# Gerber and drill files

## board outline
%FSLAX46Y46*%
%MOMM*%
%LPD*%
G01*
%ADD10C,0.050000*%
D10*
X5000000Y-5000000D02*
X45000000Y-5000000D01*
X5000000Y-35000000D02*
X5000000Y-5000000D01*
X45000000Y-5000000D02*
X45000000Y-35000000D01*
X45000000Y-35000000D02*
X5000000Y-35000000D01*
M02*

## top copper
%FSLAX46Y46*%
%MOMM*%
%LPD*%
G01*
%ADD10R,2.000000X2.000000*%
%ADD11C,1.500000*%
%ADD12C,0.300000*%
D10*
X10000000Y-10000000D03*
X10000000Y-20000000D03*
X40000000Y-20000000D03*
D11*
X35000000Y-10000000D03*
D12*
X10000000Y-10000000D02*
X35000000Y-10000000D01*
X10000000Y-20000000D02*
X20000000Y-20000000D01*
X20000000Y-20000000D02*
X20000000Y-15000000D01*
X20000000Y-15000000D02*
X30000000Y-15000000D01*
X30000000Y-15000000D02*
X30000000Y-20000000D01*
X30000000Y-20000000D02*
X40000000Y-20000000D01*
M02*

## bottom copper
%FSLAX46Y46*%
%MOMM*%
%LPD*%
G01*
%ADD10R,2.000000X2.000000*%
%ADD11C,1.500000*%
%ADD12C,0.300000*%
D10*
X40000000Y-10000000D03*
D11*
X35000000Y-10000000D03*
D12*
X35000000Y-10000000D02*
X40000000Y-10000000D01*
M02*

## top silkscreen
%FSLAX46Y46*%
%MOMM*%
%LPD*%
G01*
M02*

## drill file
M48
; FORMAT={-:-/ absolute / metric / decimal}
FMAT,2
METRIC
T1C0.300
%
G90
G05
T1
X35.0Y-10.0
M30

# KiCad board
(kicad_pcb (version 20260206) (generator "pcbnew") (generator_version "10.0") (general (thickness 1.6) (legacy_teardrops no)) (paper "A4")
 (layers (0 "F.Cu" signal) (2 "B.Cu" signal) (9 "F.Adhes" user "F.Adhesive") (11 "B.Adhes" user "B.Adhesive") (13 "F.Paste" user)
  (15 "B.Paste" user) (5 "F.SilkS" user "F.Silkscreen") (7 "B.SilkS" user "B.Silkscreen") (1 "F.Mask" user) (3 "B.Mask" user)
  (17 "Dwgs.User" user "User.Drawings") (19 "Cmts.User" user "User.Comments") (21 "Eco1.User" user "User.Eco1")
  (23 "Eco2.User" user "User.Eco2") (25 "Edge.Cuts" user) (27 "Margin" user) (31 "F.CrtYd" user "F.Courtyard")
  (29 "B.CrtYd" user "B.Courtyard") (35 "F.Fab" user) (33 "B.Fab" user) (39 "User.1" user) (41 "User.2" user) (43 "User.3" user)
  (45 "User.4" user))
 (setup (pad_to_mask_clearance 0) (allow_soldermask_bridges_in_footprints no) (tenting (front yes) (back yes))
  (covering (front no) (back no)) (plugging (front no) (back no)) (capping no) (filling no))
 (gr_line (start 5 5) (end 45 5) (stroke (width 0.05) (type default)) (layer "Edge.Cuts"))
 (gr_line (start 5 35) (end 5 5) (stroke (width 0.05) (type default)) (layer "Edge.Cuts"))
 (gr_line (start 45 5) (end 45 35) (stroke (width 0.05) (type default)) (layer "Edge.Cuts"))
 (gr_line (start 45 35) (end 5 35) (stroke (width 0.05) (type default)) (layer "Edge.Cuts"))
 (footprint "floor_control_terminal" (layer "F.Cu") (at 10 10)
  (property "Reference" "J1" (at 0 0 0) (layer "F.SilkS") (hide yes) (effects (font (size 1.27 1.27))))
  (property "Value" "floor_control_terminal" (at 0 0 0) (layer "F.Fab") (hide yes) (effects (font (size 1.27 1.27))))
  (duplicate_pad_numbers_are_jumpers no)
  (pad "1" smd rect (at 0 0) (size 2 2) (layers "F.Cu" "F.Paste" "F.Mask") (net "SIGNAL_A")))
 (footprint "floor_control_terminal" (layer "B.Cu") (at 40 10)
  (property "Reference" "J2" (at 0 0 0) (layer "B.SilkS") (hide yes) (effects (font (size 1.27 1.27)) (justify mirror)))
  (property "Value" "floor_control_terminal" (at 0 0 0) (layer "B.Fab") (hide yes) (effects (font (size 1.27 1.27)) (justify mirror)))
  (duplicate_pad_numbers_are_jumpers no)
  (pad "1" smd rect (at 0 0) (size 2 2) (layers "B.Cu" "B.Paste" "B.Mask") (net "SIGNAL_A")))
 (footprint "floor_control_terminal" (layer "F.Cu") (at 10 20)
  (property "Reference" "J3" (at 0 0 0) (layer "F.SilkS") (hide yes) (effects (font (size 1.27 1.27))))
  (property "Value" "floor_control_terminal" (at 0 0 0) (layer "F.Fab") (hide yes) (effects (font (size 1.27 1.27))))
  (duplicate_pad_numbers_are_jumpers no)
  (pad "1" smd rect (at 0 0) (size 2 2) (layers "F.Cu" "F.Paste" "F.Mask") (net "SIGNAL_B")))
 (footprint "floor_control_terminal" (layer "F.Cu") (at 40 20)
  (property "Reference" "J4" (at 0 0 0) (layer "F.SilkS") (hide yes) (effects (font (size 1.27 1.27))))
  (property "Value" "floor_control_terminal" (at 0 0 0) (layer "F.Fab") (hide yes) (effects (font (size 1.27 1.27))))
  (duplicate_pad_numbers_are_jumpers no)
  (pad "1" smd rect (at 0 0) (size 2 2) (layers "F.Cu" "F.Paste" "F.Mask") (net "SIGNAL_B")))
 (segment (start 10 10) (end 35 10) (width 0.3) (layer "F.Cu") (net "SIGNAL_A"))
 (segment (start 35 10) (end 40 10) (width 0.3) (layer "B.Cu") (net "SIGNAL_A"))
 (via (at 35 10) (size 1.5) (drill 0.3) (layers "F.Cu" "B.Cu") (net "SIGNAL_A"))
 (segment (start 10 20) (end 20 20) (width 0.3) (layer "F.Cu") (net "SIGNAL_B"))
 (segment (start 20 20) (end 20 15) (width 0.3) (layer "F.Cu") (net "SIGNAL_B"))
 (segment (start 20 15) (end 30 15) (width 0.3) (layer "F.Cu") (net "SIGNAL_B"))
 (segment (start 30 15) (end 30 20) (width 0.3) (layer "F.Cu") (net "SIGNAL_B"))
 (segment (start 30 20) (end 40 20) (width 0.3) (layer "F.Cu") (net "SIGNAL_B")))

